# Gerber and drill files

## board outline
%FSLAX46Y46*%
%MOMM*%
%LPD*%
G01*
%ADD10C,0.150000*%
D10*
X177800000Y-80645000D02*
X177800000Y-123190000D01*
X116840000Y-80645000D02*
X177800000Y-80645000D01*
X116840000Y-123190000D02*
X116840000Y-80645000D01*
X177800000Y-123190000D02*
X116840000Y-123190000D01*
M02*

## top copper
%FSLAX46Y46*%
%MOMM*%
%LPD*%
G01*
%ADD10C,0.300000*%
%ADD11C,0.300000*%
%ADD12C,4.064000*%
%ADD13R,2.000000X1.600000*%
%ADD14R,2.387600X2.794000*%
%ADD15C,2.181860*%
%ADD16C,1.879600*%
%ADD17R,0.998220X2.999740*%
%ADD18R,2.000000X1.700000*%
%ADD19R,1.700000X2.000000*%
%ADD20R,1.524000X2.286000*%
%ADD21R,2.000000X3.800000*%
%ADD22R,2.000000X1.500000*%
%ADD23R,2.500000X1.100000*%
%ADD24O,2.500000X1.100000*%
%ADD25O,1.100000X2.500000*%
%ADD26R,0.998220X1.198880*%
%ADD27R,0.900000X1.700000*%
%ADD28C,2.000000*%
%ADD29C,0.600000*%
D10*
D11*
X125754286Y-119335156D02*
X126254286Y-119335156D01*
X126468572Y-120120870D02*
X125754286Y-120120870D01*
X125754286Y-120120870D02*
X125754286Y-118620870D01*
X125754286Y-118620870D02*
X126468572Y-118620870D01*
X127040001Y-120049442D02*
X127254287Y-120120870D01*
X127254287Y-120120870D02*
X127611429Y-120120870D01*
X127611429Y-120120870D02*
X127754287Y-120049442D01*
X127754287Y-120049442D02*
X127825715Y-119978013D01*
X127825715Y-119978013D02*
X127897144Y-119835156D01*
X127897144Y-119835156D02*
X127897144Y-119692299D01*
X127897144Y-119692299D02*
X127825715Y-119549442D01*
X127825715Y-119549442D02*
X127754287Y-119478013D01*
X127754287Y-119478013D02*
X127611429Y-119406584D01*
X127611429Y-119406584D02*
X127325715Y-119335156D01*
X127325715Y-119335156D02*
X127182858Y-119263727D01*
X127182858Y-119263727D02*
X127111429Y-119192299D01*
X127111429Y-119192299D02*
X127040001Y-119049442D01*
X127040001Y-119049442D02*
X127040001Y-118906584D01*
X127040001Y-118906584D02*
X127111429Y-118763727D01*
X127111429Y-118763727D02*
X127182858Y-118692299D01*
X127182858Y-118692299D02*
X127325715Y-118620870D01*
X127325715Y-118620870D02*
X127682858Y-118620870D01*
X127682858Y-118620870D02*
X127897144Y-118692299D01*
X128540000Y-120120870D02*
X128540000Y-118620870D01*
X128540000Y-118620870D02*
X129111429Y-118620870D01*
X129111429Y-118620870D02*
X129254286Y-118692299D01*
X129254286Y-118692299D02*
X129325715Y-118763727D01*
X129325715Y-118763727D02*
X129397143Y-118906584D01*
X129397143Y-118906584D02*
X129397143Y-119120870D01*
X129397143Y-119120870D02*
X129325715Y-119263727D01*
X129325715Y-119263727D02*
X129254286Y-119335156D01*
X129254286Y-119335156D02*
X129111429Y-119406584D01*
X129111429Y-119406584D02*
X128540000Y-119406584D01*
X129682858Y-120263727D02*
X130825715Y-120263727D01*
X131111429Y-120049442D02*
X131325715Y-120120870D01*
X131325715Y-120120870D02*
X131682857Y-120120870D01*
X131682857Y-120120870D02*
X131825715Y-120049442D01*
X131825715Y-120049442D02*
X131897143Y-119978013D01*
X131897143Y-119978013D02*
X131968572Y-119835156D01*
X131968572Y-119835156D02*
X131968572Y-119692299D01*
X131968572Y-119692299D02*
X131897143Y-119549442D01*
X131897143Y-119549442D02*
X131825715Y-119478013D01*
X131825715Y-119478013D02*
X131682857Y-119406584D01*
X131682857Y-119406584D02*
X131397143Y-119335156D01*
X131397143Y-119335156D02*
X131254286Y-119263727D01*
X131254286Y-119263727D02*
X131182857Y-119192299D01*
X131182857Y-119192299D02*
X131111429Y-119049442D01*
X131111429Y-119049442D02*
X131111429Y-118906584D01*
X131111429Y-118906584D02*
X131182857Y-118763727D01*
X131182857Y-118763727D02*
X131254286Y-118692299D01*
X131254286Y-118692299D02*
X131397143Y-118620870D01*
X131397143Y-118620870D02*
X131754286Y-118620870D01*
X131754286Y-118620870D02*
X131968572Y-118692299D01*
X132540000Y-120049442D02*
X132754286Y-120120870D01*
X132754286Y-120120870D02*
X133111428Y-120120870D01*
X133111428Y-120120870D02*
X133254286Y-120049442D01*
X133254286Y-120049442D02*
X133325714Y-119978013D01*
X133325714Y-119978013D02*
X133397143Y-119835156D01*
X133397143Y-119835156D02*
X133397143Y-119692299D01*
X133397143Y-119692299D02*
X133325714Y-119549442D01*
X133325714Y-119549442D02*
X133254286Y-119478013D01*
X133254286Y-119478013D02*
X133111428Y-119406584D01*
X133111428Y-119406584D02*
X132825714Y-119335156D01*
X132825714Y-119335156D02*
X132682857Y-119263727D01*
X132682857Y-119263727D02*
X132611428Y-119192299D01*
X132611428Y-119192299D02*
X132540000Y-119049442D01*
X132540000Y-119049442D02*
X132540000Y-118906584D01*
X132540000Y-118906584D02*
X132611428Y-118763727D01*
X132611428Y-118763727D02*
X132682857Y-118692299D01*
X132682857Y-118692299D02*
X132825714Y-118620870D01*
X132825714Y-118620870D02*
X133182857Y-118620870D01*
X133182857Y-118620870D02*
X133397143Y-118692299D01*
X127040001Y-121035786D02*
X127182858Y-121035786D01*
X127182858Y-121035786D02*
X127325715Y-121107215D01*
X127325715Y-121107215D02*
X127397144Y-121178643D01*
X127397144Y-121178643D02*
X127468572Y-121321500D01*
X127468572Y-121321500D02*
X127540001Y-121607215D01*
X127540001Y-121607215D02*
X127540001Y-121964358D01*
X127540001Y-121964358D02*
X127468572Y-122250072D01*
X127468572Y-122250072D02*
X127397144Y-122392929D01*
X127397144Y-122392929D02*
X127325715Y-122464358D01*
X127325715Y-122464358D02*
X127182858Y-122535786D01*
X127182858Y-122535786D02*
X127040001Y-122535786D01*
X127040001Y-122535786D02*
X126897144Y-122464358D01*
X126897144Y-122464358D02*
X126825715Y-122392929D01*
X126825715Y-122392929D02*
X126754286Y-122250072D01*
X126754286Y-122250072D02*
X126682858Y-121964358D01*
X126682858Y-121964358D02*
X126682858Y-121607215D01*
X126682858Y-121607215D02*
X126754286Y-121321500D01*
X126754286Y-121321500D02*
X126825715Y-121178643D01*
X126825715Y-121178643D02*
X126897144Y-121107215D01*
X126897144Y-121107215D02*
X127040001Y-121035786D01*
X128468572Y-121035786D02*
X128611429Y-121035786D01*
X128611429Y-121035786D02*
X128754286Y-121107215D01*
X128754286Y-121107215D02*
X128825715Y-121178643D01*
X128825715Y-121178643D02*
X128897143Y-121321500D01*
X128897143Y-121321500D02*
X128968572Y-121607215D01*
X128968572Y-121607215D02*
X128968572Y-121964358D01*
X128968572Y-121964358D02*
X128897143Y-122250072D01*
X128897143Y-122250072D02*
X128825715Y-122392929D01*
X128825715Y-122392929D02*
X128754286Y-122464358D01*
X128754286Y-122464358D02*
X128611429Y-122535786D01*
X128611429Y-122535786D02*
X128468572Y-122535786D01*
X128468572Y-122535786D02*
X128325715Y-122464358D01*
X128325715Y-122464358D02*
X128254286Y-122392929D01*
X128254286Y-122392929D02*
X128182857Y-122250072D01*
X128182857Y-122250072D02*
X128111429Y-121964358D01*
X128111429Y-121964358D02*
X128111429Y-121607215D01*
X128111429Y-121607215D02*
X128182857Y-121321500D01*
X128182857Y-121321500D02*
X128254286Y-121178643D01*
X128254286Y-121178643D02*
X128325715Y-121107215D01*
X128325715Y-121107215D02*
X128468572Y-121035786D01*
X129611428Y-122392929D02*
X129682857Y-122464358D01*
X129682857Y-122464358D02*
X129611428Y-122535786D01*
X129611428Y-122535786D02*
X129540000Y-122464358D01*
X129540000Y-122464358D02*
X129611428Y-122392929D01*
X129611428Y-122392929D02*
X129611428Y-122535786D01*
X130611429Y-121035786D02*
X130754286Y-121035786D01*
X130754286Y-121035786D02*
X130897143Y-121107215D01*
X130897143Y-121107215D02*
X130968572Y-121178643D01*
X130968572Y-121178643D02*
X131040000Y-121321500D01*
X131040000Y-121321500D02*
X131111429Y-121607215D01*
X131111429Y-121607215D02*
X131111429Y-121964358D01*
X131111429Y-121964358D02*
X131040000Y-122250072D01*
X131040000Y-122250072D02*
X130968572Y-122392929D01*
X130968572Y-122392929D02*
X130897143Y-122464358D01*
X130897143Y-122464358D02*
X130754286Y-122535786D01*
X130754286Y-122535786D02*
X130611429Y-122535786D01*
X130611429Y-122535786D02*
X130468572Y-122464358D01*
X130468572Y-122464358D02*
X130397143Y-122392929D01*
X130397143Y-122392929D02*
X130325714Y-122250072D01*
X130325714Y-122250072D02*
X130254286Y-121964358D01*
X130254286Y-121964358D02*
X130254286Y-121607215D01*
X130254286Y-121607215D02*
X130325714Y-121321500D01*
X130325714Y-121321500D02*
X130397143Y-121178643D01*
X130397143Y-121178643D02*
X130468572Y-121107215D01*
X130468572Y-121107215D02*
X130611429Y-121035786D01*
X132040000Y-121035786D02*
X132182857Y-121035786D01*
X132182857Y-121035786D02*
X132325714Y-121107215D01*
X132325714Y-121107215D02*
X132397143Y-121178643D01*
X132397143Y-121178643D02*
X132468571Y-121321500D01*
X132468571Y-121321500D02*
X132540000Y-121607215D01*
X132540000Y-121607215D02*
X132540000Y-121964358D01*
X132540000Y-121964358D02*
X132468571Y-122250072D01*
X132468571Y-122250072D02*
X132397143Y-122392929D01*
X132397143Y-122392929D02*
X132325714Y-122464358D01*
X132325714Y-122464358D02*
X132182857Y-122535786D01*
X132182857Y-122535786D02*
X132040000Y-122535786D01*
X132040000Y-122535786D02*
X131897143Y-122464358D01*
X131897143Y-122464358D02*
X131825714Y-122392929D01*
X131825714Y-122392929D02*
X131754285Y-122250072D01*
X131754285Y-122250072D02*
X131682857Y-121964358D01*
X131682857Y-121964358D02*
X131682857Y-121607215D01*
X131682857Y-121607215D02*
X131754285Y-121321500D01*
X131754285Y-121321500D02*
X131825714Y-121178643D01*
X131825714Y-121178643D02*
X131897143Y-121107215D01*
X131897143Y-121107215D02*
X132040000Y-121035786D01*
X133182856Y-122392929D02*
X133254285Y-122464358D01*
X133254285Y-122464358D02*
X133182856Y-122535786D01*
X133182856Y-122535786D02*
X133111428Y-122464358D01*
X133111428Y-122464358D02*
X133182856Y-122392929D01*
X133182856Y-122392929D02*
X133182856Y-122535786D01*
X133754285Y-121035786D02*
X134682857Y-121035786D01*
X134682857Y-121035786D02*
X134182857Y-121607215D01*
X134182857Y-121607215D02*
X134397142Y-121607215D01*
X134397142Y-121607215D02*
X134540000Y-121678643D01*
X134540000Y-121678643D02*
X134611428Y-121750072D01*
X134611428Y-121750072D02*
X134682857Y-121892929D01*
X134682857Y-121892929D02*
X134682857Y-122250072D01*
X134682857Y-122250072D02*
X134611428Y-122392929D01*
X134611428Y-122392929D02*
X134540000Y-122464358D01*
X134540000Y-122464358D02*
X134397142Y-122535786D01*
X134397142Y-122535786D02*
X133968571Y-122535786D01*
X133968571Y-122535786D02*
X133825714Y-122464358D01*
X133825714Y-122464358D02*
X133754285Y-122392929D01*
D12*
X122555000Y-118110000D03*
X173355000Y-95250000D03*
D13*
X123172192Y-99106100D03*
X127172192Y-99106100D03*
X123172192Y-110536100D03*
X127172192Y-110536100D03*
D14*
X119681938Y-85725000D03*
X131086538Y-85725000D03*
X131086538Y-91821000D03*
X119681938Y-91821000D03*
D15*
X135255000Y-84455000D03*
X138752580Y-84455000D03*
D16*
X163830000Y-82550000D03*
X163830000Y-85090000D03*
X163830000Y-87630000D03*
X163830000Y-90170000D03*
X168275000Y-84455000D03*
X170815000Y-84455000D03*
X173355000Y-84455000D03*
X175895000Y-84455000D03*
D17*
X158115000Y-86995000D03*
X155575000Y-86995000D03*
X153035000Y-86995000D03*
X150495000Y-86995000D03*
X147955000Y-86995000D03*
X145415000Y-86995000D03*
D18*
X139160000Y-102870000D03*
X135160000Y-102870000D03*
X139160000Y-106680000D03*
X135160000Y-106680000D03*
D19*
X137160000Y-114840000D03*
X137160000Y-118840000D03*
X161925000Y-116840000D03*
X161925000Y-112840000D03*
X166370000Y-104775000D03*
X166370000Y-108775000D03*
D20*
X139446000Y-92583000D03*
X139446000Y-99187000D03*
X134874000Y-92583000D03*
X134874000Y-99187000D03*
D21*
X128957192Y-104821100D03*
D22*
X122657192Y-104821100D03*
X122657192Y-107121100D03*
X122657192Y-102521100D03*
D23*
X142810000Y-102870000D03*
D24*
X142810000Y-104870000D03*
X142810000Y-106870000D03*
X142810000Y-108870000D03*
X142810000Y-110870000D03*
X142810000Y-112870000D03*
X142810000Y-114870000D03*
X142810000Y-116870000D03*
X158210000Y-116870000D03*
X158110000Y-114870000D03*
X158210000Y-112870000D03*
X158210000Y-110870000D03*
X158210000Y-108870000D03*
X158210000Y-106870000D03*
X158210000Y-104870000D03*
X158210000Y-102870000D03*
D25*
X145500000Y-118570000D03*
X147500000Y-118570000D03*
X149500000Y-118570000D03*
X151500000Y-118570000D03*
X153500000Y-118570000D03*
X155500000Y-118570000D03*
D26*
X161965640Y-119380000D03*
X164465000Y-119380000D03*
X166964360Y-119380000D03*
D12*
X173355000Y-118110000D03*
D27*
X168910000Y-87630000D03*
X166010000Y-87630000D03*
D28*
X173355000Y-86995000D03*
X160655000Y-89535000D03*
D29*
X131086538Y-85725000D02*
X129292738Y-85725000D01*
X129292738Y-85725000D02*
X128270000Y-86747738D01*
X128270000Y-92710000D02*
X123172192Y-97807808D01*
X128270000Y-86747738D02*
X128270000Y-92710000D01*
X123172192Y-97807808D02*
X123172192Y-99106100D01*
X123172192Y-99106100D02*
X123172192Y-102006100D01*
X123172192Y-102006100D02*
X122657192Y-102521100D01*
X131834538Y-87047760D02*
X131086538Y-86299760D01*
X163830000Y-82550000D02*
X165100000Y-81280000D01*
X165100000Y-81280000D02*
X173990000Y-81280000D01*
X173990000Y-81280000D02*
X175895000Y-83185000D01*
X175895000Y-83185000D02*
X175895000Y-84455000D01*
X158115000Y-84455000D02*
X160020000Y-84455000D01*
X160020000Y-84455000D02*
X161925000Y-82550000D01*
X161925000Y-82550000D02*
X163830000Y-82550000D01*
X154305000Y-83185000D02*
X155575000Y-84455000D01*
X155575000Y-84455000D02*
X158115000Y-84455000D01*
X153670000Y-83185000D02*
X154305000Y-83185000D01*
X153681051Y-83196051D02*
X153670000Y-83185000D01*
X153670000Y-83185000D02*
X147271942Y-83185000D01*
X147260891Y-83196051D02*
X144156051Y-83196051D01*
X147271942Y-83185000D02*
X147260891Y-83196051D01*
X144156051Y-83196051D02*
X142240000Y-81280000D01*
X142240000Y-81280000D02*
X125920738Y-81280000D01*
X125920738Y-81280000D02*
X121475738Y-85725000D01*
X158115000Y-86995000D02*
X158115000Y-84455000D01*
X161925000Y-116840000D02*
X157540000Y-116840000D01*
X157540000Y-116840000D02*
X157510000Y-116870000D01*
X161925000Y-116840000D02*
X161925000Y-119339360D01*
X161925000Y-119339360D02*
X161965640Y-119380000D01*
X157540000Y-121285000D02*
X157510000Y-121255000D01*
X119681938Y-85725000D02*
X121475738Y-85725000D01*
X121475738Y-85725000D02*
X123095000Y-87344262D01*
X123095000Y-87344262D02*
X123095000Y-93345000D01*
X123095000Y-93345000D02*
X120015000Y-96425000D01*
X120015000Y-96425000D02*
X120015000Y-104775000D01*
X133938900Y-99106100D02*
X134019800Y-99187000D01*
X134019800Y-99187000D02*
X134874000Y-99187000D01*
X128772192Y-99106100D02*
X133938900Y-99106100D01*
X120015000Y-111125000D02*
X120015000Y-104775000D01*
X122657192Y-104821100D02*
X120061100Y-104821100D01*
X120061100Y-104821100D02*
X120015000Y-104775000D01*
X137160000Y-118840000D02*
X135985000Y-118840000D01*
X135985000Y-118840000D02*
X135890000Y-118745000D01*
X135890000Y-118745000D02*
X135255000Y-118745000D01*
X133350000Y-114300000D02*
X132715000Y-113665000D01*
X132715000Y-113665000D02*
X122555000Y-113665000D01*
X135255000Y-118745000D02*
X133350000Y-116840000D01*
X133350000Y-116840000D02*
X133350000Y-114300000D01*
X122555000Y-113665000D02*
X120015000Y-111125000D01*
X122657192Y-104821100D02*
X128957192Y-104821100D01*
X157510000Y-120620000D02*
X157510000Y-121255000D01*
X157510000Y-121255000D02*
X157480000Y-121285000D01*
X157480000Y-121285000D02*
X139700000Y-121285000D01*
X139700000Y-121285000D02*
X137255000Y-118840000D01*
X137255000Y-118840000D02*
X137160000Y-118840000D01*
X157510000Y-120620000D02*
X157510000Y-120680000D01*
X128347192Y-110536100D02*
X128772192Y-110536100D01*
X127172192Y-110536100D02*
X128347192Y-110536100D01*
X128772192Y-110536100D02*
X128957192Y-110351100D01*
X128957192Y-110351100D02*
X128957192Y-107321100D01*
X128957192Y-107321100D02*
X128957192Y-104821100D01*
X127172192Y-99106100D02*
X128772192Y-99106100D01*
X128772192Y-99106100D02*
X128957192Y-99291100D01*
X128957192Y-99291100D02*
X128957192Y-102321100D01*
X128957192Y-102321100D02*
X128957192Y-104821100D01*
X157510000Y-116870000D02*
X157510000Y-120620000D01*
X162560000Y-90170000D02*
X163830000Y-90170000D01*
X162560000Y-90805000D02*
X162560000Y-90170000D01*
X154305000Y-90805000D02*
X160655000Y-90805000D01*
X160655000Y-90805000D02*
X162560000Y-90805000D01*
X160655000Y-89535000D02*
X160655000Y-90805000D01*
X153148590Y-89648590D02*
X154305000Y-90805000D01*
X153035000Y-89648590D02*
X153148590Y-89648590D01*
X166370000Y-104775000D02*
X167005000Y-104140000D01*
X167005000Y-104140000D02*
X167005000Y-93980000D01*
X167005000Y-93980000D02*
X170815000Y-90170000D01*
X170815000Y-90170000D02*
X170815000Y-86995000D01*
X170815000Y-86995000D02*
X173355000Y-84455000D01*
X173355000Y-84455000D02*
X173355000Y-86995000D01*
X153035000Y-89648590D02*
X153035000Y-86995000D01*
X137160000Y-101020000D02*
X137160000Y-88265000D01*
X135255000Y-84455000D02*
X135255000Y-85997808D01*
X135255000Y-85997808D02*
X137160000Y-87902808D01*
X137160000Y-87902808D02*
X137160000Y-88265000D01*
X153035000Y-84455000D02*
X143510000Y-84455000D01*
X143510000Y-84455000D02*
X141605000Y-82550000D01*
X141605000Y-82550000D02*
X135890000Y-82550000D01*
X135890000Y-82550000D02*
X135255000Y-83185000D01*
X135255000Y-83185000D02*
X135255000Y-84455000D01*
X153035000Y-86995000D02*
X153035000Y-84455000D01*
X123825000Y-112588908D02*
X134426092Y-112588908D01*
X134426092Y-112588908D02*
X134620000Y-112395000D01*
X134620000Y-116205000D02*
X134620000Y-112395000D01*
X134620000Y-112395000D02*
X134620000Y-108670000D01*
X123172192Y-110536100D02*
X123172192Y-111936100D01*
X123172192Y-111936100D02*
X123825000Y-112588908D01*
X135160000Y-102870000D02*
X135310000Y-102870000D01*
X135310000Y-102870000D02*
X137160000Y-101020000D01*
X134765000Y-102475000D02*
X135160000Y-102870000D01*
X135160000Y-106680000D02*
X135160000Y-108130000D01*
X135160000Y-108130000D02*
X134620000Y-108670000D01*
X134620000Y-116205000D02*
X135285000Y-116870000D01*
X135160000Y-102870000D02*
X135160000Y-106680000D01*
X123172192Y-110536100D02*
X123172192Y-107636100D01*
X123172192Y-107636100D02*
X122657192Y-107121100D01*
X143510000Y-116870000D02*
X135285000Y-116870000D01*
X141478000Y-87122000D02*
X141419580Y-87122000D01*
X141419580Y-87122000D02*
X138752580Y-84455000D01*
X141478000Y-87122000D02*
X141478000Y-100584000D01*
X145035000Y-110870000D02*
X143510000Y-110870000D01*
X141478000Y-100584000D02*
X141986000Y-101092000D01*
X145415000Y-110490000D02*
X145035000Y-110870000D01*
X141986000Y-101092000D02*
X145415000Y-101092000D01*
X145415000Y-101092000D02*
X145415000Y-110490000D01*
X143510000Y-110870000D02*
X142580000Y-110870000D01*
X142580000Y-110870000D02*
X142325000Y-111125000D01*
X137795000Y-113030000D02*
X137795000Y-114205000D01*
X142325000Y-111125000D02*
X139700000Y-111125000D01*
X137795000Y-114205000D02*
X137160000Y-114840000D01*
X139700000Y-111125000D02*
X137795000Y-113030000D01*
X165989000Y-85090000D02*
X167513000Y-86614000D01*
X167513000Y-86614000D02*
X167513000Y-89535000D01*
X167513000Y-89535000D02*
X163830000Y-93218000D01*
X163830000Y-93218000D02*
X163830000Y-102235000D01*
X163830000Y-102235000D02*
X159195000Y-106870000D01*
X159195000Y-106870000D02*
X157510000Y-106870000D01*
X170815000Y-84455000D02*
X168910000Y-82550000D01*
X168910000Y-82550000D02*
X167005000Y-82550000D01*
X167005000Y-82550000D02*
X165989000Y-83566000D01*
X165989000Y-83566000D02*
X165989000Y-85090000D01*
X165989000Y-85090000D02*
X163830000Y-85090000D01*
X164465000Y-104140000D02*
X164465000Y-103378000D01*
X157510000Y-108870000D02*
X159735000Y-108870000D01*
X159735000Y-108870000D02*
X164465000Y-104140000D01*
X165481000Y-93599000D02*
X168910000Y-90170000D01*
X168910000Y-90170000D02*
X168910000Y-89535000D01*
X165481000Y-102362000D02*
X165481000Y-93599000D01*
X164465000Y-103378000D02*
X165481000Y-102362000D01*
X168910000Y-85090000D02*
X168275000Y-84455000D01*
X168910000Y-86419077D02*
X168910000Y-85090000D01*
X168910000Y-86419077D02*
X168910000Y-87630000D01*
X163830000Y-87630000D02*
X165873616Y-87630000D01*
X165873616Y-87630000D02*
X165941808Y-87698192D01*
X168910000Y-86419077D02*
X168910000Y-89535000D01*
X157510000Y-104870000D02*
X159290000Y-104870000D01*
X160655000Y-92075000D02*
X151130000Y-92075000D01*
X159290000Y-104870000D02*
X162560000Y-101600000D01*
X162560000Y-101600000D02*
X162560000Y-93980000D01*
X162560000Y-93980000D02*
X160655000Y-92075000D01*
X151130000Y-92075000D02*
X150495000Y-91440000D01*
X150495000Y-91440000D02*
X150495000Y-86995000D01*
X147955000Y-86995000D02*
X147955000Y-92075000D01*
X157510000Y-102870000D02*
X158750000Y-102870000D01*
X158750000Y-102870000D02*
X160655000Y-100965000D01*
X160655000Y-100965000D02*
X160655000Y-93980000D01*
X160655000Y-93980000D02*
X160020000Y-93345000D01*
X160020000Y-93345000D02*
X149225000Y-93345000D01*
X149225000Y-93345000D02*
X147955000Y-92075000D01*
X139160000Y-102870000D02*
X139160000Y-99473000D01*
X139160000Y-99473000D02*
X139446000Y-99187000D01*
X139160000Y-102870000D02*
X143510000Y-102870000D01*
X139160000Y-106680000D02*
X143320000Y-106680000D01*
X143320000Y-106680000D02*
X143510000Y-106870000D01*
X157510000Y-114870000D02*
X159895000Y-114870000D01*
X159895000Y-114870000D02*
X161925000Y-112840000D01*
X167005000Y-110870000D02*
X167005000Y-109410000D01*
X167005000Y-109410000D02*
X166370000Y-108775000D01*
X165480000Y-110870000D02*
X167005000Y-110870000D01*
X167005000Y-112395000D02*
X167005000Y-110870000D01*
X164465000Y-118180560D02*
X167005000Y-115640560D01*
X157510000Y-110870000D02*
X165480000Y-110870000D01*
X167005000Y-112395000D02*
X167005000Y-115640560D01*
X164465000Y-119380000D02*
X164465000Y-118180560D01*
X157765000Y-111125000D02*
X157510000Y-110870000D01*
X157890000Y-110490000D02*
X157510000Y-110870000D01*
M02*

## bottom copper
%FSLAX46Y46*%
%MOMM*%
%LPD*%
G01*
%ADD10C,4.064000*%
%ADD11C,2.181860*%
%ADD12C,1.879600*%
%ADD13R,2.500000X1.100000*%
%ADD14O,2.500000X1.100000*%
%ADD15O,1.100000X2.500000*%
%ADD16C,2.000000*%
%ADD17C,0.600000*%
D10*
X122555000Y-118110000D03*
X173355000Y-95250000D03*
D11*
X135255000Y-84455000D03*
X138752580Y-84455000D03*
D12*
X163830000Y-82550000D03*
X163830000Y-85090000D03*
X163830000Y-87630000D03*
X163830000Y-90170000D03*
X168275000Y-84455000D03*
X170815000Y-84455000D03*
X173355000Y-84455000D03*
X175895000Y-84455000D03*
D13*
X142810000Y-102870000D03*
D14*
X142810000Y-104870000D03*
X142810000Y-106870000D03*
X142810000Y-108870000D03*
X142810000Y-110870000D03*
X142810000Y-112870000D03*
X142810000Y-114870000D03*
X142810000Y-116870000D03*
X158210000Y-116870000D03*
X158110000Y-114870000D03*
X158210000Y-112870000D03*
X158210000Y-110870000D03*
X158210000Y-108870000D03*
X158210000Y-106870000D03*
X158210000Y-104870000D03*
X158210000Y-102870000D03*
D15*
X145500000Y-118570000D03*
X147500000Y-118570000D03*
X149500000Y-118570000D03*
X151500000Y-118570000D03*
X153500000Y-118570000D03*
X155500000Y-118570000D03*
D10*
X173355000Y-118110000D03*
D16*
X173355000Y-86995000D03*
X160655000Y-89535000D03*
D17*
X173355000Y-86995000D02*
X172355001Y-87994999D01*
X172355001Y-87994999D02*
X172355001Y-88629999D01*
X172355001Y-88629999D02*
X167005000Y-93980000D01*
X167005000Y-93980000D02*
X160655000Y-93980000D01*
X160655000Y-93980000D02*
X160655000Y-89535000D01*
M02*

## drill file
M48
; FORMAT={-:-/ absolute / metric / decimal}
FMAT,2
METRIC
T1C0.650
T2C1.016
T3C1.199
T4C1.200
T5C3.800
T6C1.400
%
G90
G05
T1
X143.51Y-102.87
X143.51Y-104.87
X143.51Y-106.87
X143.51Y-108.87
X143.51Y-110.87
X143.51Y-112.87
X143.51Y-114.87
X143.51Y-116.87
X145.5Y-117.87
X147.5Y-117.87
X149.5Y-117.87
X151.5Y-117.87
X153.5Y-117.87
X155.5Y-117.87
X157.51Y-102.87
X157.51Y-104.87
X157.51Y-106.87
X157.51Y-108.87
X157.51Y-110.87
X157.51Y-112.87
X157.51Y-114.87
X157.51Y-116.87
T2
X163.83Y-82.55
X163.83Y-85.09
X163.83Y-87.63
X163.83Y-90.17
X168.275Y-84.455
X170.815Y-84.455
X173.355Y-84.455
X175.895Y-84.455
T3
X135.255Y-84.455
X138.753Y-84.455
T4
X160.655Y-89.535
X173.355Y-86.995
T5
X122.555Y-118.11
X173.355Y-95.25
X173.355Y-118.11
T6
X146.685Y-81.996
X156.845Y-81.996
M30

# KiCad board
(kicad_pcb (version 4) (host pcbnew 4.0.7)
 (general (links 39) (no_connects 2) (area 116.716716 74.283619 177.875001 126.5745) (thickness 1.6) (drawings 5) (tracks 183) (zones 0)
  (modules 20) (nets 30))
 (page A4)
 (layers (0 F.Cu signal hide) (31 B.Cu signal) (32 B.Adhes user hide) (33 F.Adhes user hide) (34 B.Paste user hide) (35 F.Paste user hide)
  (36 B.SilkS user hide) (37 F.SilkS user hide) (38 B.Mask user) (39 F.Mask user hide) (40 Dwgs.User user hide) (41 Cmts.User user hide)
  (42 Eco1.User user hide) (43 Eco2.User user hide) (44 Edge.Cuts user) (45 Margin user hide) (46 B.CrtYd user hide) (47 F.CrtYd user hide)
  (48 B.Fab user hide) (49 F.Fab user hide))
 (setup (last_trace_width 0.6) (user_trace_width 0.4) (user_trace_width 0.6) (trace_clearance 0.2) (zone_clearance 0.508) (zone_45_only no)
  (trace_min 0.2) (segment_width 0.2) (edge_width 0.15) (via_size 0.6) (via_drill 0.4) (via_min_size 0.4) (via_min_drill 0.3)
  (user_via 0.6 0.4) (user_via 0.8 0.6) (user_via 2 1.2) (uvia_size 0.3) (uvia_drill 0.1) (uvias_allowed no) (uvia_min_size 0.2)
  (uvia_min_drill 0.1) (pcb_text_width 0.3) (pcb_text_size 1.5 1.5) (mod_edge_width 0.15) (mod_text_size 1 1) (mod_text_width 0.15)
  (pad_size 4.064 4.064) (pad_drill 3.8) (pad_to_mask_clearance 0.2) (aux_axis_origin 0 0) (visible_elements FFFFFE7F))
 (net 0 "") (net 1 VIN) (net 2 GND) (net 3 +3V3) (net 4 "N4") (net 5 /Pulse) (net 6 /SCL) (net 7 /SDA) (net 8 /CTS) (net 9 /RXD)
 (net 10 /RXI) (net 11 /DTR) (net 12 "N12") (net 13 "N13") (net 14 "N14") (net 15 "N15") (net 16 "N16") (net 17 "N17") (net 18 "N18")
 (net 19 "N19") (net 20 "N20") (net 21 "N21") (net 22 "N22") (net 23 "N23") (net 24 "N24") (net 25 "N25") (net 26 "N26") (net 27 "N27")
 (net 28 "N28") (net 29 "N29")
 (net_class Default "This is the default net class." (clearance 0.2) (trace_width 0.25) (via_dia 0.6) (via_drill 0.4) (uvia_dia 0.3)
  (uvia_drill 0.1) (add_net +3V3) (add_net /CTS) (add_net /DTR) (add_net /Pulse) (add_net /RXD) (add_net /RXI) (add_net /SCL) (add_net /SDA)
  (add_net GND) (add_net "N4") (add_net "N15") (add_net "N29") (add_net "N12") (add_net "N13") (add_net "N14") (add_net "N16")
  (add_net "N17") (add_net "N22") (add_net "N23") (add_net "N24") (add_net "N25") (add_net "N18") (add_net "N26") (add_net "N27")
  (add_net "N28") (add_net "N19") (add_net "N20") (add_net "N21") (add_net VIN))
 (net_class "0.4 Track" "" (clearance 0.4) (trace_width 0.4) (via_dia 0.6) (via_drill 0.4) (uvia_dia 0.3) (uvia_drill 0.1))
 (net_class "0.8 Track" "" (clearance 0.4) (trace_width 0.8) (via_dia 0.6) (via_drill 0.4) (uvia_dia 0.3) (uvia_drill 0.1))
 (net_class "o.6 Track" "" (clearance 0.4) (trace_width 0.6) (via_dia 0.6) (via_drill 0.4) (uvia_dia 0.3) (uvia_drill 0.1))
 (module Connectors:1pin (layer F.Cu) (at 122.555 118.11)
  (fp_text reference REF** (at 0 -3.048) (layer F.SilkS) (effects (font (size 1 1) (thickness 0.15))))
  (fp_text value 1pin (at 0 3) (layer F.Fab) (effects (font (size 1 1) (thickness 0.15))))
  (pad 1 thru_hole circle (at 0 0) (size 4.064 4.064) (drill 3.8) (layers *.Cu *.Mask)))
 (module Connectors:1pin (layer F.Cu) (at 173.355 95.25)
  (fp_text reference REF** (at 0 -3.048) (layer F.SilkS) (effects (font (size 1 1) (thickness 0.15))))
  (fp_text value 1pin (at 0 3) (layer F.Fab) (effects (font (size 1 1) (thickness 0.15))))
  (pad 1 thru_hole circle (at 0 0) (size 4.064 4.064) (drill 3.8) (layers *.Cu *.Mask)))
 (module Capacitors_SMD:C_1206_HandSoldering (layer F.Cu) (at 125.172192 99.1061)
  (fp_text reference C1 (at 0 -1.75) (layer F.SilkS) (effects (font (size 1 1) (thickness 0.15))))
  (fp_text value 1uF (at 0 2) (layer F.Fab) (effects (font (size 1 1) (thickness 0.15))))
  (pad 1 smd rect (at -2 0) (size 2 1.6) (layers F.Cu F.Paste F.Mask) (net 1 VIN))
  (pad 2 smd rect (at 2 0) (size 2 1.6) (layers F.Cu F.Paste F.Mask) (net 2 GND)))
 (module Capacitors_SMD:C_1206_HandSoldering (layer F.Cu) (at 125.172192 110.5361)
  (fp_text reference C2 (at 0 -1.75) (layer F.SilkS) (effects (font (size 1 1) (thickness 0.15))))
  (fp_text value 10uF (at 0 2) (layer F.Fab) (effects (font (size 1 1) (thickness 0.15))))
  (pad 1 smd rect (at -2 0) (size 2 1.6) (layers F.Cu F.Paste F.Mask) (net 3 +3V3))
  (pad 2 smd rect (at 2 0) (size 2 1.6) (layers F.Cu F.Paste F.Mask) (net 2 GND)))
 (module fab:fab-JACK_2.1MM (layer F.Cu) (at 125.447738 88.138 180)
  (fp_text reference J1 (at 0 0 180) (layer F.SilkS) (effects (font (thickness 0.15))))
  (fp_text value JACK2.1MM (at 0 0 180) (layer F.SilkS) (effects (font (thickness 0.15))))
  (pad CONT smd rect (at 5.7658 2.413 180) (size 2.3876 2.794) (layers F.Cu F.Paste F.Mask) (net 2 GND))
  (pad PIN smd rect (at -5.6388 2.413 180) (size 2.3876 2.794) (layers F.Cu F.Paste F.Mask) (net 1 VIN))
  (pad PIN1 smd rect (at -5.6388 -3.683 180) (size 2.3876 2.794) (layers F.Cu F.Paste F.Mask))
  (pad SHUN smd rect (at 5.7658 -3.683 180) (size 2.3876 2.794) (layers F.Cu F.Paste F.Mask) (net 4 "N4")))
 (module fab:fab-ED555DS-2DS (layer F.Cu) (at 137.05332 84.455 180)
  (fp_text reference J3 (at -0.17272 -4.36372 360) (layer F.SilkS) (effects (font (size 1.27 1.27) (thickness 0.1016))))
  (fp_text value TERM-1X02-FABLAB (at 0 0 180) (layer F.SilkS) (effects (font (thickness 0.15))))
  (pad 1 thru_hole circle (at 1.79832 0 180) (size 2.18186 2.18186) (drill 1.19888) (layers *.Cu F.Paste F.SilkS F.Mask) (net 3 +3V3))
  (pad 2 thru_hole circle (at -1.69926 0 180) (size 2.18186 2.18186) (drill 1.19888) (layers *.Cu F.Paste F.SilkS F.Mask) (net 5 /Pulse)))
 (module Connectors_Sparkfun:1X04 (layer F.Cu) (at 163.83 82.55 270)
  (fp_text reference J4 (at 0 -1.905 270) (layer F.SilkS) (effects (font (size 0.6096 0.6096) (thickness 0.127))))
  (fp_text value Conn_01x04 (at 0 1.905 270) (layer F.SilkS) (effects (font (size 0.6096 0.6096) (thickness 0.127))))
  (pad 1 thru_hole circle (at 0 0 270) (size 1.8796 1.8796) (drill 1.016) (layers *.Cu *.Mask) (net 2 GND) (solder_mask_margin 0.1016))
  (pad 2 thru_hole circle (at 2.54 0 270) (size 1.8796 1.8796) (drill 1.016) (layers *.Cu *.Mask) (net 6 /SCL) (solder_mask_margin 0.1016))
  (pad 3 thru_hole circle (at 5.08 0 270) (size 1.8796 1.8796) (drill 1.016) (layers *.Cu *.Mask) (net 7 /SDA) (solder_mask_margin 0.1016))
  (pad 4 thru_hole circle (at 7.62 0 270) (size 1.8796 1.8796) (drill 1.016) (layers *.Cu *.Mask) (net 3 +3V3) (solder_mask_margin 0.1016)))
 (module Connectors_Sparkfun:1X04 (layer F.Cu) (at 168.275 84.455)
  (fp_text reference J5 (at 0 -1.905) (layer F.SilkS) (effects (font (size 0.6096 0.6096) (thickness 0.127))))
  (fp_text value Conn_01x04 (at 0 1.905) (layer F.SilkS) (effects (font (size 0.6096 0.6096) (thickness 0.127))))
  (pad 1 thru_hole circle (at 0 0) (size 1.8796 1.8796) (drill 1.016) (layers *.Cu *.Mask) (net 7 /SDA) (solder_mask_margin 0.1016))
  (pad 2 thru_hole circle (at 2.54 0) (size 1.8796 1.8796) (drill 1.016) (layers *.Cu *.Mask) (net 6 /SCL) (solder_mask_margin 0.1016))
  (pad 3 thru_hole circle (at 5.08 0) (size 1.8796 1.8796) (drill 1.016) (layers *.Cu *.Mask) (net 3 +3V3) (solder_mask_margin 0.1016))
  (pad 4 thru_hole circle (at 7.62 0) (size 1.8796 1.8796) (drill 1.016) (layers *.Cu *.Mask) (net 2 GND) (solder_mask_margin 0.1016)))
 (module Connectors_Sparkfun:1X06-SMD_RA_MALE (layer F.Cu) (at 151.765 81.99628 180)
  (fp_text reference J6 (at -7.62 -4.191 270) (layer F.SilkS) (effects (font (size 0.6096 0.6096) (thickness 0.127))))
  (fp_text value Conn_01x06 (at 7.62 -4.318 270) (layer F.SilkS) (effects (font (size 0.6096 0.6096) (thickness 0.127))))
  (pad 1 smd rect (at -6.35 -4.99872 270) (size 2.99974 0.99822) (layers F.Cu F.Paste F.Mask) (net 2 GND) (solder_mask_margin 0.1016))
  (pad 2 smd rect (at -3.81 -4.99872 270) (size 2.99974 0.99822) (layers F.Cu F.Paste F.Mask) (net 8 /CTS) (solder_mask_margin 0.1016))
  (pad 3 smd rect (at -1.27 -4.99872 270) (size 2.99974 0.99822) (layers F.Cu F.Paste F.Mask) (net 3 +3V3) (solder_mask_margin 0.1016))
  (pad 4 smd rect (at 1.27 -4.99872 270) (size 2.99974 0.99822) (layers F.Cu F.Paste F.Mask) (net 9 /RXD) (solder_mask_margin 0.1016))
  (pad 5 smd rect (at 3.81 -4.99872 270) (size 2.99974 0.99822) (layers F.Cu F.Paste F.Mask) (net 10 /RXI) (solder_mask_margin 0.1016))
  (pad 6 smd rect (at 6.35 -4.99872 270) (size 2.99974 0.99822) (layers F.Cu F.Paste F.Mask) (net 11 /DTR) (solder_mask_margin 0.1016))
  (pad "" np_thru_hole circle (at -5.08 0 180) (size 1.39954 1.39954) (drill 1.39954) (layers *.Cu *.Mask) (solder_mask_margin 0.1016))
  (pad "" np_thru_hole circle (at 5.08 0 180) (size 1.39954 1.39954) (drill 1.39954) (layers *.Cu *.Mask) (solder_mask_margin 0.1016)))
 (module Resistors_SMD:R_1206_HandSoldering (layer F.Cu) (at 137.16 102.87 180)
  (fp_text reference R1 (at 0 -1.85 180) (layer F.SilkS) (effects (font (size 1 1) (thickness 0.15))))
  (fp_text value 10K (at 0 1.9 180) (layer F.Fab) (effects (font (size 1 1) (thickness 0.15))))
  (pad 1 smd rect (at -2 0 180) (size 2 1.7) (layers F.Cu F.Paste F.Mask) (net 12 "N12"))
  (pad 2 smd rect (at 2 0 180) (size 2 1.7) (layers F.Cu F.Paste F.Mask) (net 3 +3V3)))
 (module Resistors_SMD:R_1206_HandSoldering (layer F.Cu) (at 137.16 106.68 180)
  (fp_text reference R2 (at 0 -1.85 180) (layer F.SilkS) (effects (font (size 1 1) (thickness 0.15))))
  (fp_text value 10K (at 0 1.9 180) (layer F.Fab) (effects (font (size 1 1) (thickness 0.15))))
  (pad 1 smd rect (at -2 0 180) (size 2 1.7) (layers F.Cu F.Paste F.Mask) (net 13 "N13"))
  (pad 2 smd rect (at 2 0 180) (size 2 1.7) (layers F.Cu F.Paste F.Mask) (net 3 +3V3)))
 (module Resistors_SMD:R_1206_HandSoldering (layer F.Cu) (at 137.16 116.84 270)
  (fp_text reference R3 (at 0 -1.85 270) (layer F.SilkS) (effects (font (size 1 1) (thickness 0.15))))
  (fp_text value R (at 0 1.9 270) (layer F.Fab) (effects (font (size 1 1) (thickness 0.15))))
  (pad 1 smd rect (at -2 0 270) (size 2 1.7) (layers F.Cu F.Paste F.Mask) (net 5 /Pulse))
  (pad 2 smd rect (at 2 0 270) (size 2 1.7) (layers F.Cu F.Paste F.Mask) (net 2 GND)))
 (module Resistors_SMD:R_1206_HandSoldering (layer F.Cu) (at 161.925 114.84 90)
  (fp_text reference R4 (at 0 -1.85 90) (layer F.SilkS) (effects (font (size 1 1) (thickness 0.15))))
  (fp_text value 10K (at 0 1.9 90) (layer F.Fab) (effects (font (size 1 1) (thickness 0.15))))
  (pad 1 smd rect (at -2 0 90) (size 2 1.7) (layers F.Cu F.Paste F.Mask) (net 2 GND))
  (pad 2 smd rect (at 2 0 90) (size 2 1.7) (layers F.Cu F.Paste F.Mask) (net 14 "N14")))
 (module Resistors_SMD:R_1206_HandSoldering (layer F.Cu) (at 166.37 106.775 270)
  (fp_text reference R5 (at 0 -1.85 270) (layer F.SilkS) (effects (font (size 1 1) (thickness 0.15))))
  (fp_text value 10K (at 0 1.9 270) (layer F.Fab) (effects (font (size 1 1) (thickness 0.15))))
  (pad 1 smd rect (at -2 0 270) (size 2 1.7) (layers F.Cu F.Paste F.Mask) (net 3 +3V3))
  (pad 2 smd rect (at 2 0 270) (size 2 1.7) (layers F.Cu F.Paste F.Mask) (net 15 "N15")))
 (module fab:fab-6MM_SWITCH (layer F.Cu) (at 137.16 95.885 270)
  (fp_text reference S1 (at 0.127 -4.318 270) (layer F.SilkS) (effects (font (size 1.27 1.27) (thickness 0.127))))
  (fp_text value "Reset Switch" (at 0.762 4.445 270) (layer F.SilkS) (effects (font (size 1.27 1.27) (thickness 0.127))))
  (pad 1 smd rect (at -3.302 -2.286 270) (size 2.286 1.524) (layers F.Cu F.Paste F.Mask) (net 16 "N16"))
  (pad 2 smd rect (at 3.302 -2.286 270) (size 2.286 1.524) (layers F.Cu F.Paste F.Mask) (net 12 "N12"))
  (pad 3 smd rect (at -3.302 2.286 270) (size 2.286 1.524) (layers F.Cu F.Paste F.Mask) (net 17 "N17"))
  (pad 4 smd rect (at 3.302 2.286 270) (size 2.286 1.524) (layers F.Cu F.Paste F.Mask) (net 2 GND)))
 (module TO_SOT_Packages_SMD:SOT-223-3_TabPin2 (layer F.Cu) (at 125.807192 104.8211)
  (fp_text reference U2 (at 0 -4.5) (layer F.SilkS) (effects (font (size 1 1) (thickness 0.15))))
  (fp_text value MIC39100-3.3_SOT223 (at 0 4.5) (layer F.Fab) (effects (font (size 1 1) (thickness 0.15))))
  (pad 2 smd rect (at 3.15 0) (size 2 3.8) (layers F.Cu F.Paste F.Mask) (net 2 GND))
  (pad 2 smd rect (at -3.15 0) (size 2 1.5) (layers F.Cu F.Paste F.Mask) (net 2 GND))
  (pad 3 smd rect (at -3.15 2.3) (size 2 1.5) (layers F.Cu F.Paste F.Mask) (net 3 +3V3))
  (pad 1 smd rect (at -3.15 -2.3) (size 2 1.5) (layers F.Cu F.Paste F.Mask) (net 1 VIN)))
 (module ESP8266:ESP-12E (layer F.Cu) (at 143.51 102.87)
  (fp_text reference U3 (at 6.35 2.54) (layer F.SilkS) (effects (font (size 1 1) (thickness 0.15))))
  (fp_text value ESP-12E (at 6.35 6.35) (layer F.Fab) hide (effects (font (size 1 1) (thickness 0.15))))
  (pad 1 thru_hole rect (at 0 0) (size 2.5 1.1) (drill 0.65 (offset -0.7 0)) (layers *.Cu *.Mask F.SilkS) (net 12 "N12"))
  (pad 2 thru_hole oval (at 0 2) (size 2.5 1.1) (drill 0.65 (offset -0.7 0)) (layers *.Cu *.Mask F.SilkS) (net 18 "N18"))
  (pad 3 thru_hole oval (at 0 4) (size 2.5 1.1) (drill 0.65 (offset -0.7 0)) (layers *.Cu *.Mask F.SilkS) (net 13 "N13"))
  (pad 4 thru_hole oval (at 0 6) (size 2.5 1.1) (drill 0.65 (offset -0.7 0)) (layers *.Cu *.Mask F.SilkS) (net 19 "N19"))
  (pad 5 thru_hole oval (at 0 8) (size 2.5 1.1) (drill 0.65 (offset -0.7 0)) (layers *.Cu *.Mask F.SilkS) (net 5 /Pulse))
  (pad 6 thru_hole oval (at 0 10) (size 2.5 1.1) (drill 0.65 (offset -0.7 0)) (layers *.Cu *.Mask F.SilkS) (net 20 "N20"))
  (pad 7 thru_hole oval (at 0 12) (size 2.5 1.1) (drill 0.65 (offset -0.7 0)) (layers *.Cu *.Mask F.SilkS) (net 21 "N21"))
  (pad 8 thru_hole oval (at 0 14) (size 2.5 1.1) (drill 0.65 (offset -0.7 0)) (layers *.Cu *.Mask F.SilkS) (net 3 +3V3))
  (pad 9 thru_hole oval (at 14 14) (size 2.5 1.1) (drill 0.65 (offset 0.7 0)) (layers *.Cu *.Mask F.SilkS) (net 2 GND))
  (pad 10 thru_hole oval (at 14 12) (size 2.5 1.1) (drill 0.65 (offset 0.6 0)) (layers *.Cu *.Mask F.SilkS) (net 14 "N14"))
  (pad 11 thru_hole oval (at 14 10) (size 2.5 1.1) (drill 0.65 (offset 0.7 0)) (layers *.Cu *.Mask F.SilkS) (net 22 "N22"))
  (pad 12 thru_hole oval (at 14 8) (size 2.5 1.1) (drill 0.65 (offset 0.7 0)) (layers *.Cu *.Mask F.SilkS) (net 15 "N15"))
  (pad 13 thru_hole oval (at 14 6) (size 2.5 1.1) (drill 0.65 (offset 0.7 0)) (layers *.Cu *.Mask F.SilkS) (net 7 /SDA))
  (pad 14 thru_hole oval (at 14 4) (size 2.5 1.1) (drill 0.65 (offset 0.7 0)) (layers *.Cu *.Mask F.SilkS) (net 6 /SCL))
  (pad 15 thru_hole oval (at 14 2) (size 2.5 1.1) (drill 0.65 (offset 0.7 0)) (layers *.Cu *.Mask F.SilkS) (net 9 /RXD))
  (pad 16 thru_hole oval (at 14 0) (size 2.5 1.1) (drill 0.65 (offset 0.7 0)) (layers *.Cu *.Mask F.SilkS) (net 10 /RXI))
  (pad 17 thru_hole oval (at 1.99 15 90) (size 2.5 1.1) (drill 0.65 (offset -0.7 0)) (layers *.Cu *.Mask F.SilkS) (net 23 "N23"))
  (pad 18 thru_hole oval (at 3.99 15 90) (size 2.5 1.1) (drill 0.65 (offset -0.7 0)) (layers *.Cu *.Mask F.SilkS) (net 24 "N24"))
  (pad 19 thru_hole oval (at 5.99 15 90) (size 2.5 1.1) (drill 0.65 (offset -0.7 0)) (layers *.Cu *.Mask F.SilkS) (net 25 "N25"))
  (pad 20 thru_hole oval (at 7.99 15 90) (size 2.5 1.1) (drill 0.65 (offset -0.7 0)) (layers *.Cu *.Mask F.SilkS) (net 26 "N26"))
  (pad 21 thru_hole oval (at 9.99 15 90) (size 2.5 1.1) (drill 0.65 (offset -0.7 0)) (layers *.Cu *.Mask F.SilkS) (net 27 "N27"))
  (pad 22 thru_hole oval (at 11.99 15 90) (size 2.5 1.1) (drill 0.65 (offset -0.7 0)) (layers *.Cu *.Mask F.SilkS) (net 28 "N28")))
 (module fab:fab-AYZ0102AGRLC (layer F.Cu) (at 164.465 121.6787 180)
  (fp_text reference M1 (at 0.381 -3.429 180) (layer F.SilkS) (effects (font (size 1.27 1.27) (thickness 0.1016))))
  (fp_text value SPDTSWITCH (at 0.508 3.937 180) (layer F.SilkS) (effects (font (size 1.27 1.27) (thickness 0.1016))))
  (pad 1 smd rect (at 2.49936 2.2987 180) (size 0.99822 1.19888) (layers F.Cu F.Paste F.Mask) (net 2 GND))
  (pad 2 smd rect (at 0 2.2987 180) (size 0.99822 1.19888) (layers F.Cu F.Paste F.Mask) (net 15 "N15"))
  (pad 3 smd rect (at -2.49936 2.2987 180) (size 0.99822 1.19888) (layers F.Cu F.Paste F.Mask) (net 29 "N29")))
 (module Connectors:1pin (layer F.Cu) (at 173.355 118.11)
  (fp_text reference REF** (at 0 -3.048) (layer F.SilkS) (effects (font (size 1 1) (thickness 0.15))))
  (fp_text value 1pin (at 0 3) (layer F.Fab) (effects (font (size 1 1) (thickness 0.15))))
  (pad 1 thru_hole circle (at 0 0) (size 4.064 4.064) (drill 3.8) (layers *.Cu *.Mask)))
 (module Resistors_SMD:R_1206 (layer F.Cu) (at 167.46 87.63 180)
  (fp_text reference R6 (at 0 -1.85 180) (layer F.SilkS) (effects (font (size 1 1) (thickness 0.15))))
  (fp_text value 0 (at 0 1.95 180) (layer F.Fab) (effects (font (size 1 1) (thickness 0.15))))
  (pad 1 smd rect (at -1.45 0 180) (size 0.9 1.7) (layers F.Cu F.Paste F.Mask) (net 7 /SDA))
  (pad 2 smd rect (at 1.45 0 180) (size 0.9 1.7) (layers F.Cu F.Paste F.Mask) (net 7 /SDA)))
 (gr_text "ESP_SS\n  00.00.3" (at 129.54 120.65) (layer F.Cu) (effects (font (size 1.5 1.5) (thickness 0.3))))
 (gr_line (start 177.8 80.645) (end 177.8 123.19) (layer Edge.Cuts) (width 0.15))
 (gr_line (start 116.84 80.645) (end 177.8 80.645) (layer Edge.Cuts) (width 0.15))
 (gr_line (start 116.84 123.19) (end 116.84 80.645) (layer Edge.Cuts) (width 0.15))
 (gr_line (start 177.8 123.19) (end 116.84 123.19) (layer Edge.Cuts) (width 0.15))
 (segment (start 131.086538 85.725) (end 129.292738 85.725) (width 0.6) (layer F.Cu) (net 1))
 (segment (start 129.292738 85.725) (end 128.27 86.747738) (width 0.6) (layer F.Cu) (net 1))
 (segment (start 128.27 92.71) (end 123.172192 97.807808) (width 0.6) (layer F.Cu) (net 1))
 (segment (start 128.27 86.747738) (end 128.27 92.71) (width 0.6) (layer F.Cu) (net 1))
 (segment (start 123.172192 97.807808) (end 123.172192 99.1061) (width 0.6) (layer F.Cu) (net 1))
 (segment (start 123.172192 99.1061) (end 123.172192 102.0061) (width 0.6) (layer F.Cu) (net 1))
 (segment (start 123.172192 102.0061) (end 122.657192 102.5211) (width 0.6) (layer F.Cu) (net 1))
 (segment (start 131.834538 87.04776) (end 131.086538 86.29976) (width 0.6) (layer F.Cu) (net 1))
 (segment (start 163.83 82.55) (end 165.1 81.28) (width 0.6) (layer F.Cu) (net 2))
 (segment (start 165.1 81.28) (end 173.99 81.28) (width 0.6) (layer F.Cu) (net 2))
 (segment (start 173.99 81.28) (end 175.895 83.185) (width 0.6) (layer F.Cu) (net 2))
 (segment (start 175.895 83.185) (end 175.895 84.455) (width 0.6) (layer F.Cu) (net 2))
 (segment (start 158.115 84.455) (end 160.02 84.455) (width 0.6) (layer F.Cu) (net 2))
 (segment (start 160.02 84.455) (end 161.925 82.55) (width 0.6) (layer F.Cu) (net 2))
 (segment (start 161.925 82.55) (end 163.83 82.55) (width 0.6) (layer F.Cu) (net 2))
 (segment (start 154.305 83.185) (end 155.575 84.455) (width 0.6) (layer F.Cu) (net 2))
 (segment (start 155.575 84.455) (end 158.115 84.455) (width 0.6) (layer F.Cu) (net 2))
 (segment (start 153.67 83.185) (end 154.305 83.185) (width 0.6) (layer F.Cu) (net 2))
 (segment (start 153.681051 83.196051) (end 153.67 83.185) (width 0.6) (layer F.Cu) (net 2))
 (segment (start 153.67 83.185) (end 147.271942 83.185) (width 0.6) (layer F.Cu) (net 2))
 (segment (start 147.260891 83.196051) (end 144.156051 83.196051) (width 0.6) (layer F.Cu) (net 2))
 (segment (start 147.271942 83.185) (end 147.260891 83.196051) (width 0.6) (layer F.Cu) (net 2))
 (segment (start 144.156051 83.196051) (end 142.24 81.28) (width 0.6) (layer F.Cu) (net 2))
 (segment (start 142.24 81.28) (end 125.920738 81.28) (width 0.6) (layer F.Cu) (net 2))
 (segment (start 125.920738 81.28) (end 121.475738 85.725) (width 0.6) (layer F.Cu) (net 2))
 (segment (start 158.115 86.995) (end 158.115 84.455) (width 0.6) (layer F.Cu) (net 2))
 (segment (start 161.925 116.84) (end 157.54 116.84) (width 0.6) (layer F.Cu) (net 2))
 (segment (start 157.54 116.84) (end 157.51 116.87) (width 0.6) (layer F.Cu) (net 2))
 (segment (start 161.925 116.84) (end 161.925 119.33936) (width 0.6) (layer F.Cu) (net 2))
 (segment (start 161.925 119.33936) (end 161.96564 119.38) (width 0.6) (layer F.Cu) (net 2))
 (segment (start 157.54 121.285) (end 157.51 121.255) (width 0.6) (layer F.Cu) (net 2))
 (segment (start 119.681938 85.725) (end 121.475738 85.725) (width 0.6) (layer F.Cu) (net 2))
 (segment (start 121.475738 85.725) (end 123.095 87.344262) (width 0.6) (layer F.Cu) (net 2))
 (segment (start 123.095 87.344262) (end 123.095 93.345) (width 0.6) (layer F.Cu) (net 2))
 (segment (start 123.095 93.345) (end 120.015 96.425) (width 0.6) (layer F.Cu) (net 2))
 (segment (start 120.015 96.425) (end 120.015 104.775) (width 0.6) (layer F.Cu) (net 2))
 (segment (start 133.9389 99.1061) (end 134.0198 99.187) (width 0.6) (layer F.Cu) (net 2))
 (segment (start 134.0198 99.187) (end 134.874 99.187) (width 0.6) (layer F.Cu) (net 2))
 (segment (start 128.772192 99.1061) (end 133.9389 99.1061) (width 0.6) (layer F.Cu) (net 2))
 (segment (start 120.015 111.125) (end 120.015 104.775) (width 0.6) (layer F.Cu) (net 2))
 (segment (start 122.657192 104.8211) (end 120.0611 104.8211) (width 0.6) (layer F.Cu) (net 2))
 (segment (start 120.0611 104.8211) (end 120.015 104.775) (width 0.6) (layer F.Cu) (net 2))
 (segment (start 137.16 118.84) (end 135.985 118.84) (width 0.6) (layer F.Cu) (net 2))
 (segment (start 135.985 118.84) (end 135.89 118.745) (width 0.6) (layer F.Cu) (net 2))
 (segment (start 135.89 118.745) (end 135.255 118.745) (width 0.6) (layer F.Cu) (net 2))
 (segment (start 133.35 114.3) (end 132.715 113.665) (width 0.6) (layer F.Cu) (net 2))
 (segment (start 132.715 113.665) (end 122.555 113.665) (width 0.6) (layer F.Cu) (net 2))
 (segment (start 135.255 118.745) (end 133.35 116.84) (width 0.6) (layer F.Cu) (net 2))
 (segment (start 133.35 116.84) (end 133.35 114.3) (width 0.6) (layer F.Cu) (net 2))
 (segment (start 122.555 113.665) (end 120.015 111.125) (width 0.6) (layer F.Cu) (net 2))
 (segment (start 122.657192 104.8211) (end 128.957192 104.8211) (width 0.6) (layer F.Cu) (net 2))
 (segment (start 157.51 120.62) (end 157.51 121.255) (width 0.6) (layer F.Cu) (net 2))
 (segment (start 157.51 121.255) (end 157.48 121.285) (width 0.6) (layer F.Cu) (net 2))
 (segment (start 157.48 121.285) (end 139.7 121.285) (width 0.6) (layer F.Cu) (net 2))
 (segment (start 139.7 121.285) (end 137.255 118.84) (width 0.6) (layer F.Cu) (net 2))
 (segment (start 137.255 118.84) (end 137.16 118.84) (width 0.6) (layer F.Cu) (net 2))
 (segment (start 157.51 120.62) (end 157.51 120.68) (width 0.6) (layer F.Cu) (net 2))
 (segment (start 128.347192 110.5361) (end 128.772192 110.5361) (width 0.6) (layer F.Cu) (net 2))
 (segment (start 127.172192 110.5361) (end 128.347192 110.5361) (width 0.6) (layer F.Cu) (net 2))
 (segment (start 128.772192 110.5361) (end 128.957192 110.3511) (width 0.6) (layer F.Cu) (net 2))
 (segment (start 128.957192 110.3511) (end 128.957192 107.3211) (width 0.6) (layer F.Cu) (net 2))
 (segment (start 128.957192 107.3211) (end 128.957192 104.8211) (width 0.6) (layer F.Cu) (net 2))
 (segment (start 127.172192 99.1061) (end 128.772192 99.1061) (width 0.6) (layer F.Cu) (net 2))
 (segment (start 128.772192 99.1061) (end 128.957192 99.2911) (width 0.6) (layer F.Cu) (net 2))
 (segment (start 128.957192 99.2911) (end 128.957192 102.3211) (width 0.6) (layer F.Cu) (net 2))
 (segment (start 128.957192 102.3211) (end 128.957192 104.8211) (width 0.6) (layer F.Cu) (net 2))
 (segment (start 157.51 116.87) (end 157.51 120.62) (width 0.6) (layer F.Cu) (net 2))
 (segment (start 162.56 90.17) (end 163.83 90.17) (width 0.6) (layer F.Cu) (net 3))
 (segment (start 162.56 90.805) (end 162.56 90.17) (width 0.6) (layer F.Cu) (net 3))
 (segment (start 154.305 90.805) (end 160.655 90.805) (width 0.6) (layer F.Cu) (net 3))
 (segment (start 160.655 90.805) (end 162.56 90.805) (width 0.6) (layer F.Cu) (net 3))
 (segment (start 160.655 89.535) (end 160.655 90.805) (width 0.6) (layer F.Cu) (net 3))
 (segment (start 153.14859 89.64859) (end 154.305 90.805) (width 0.6) (layer F.Cu) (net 3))
 (segment (start 153.035 89.64859) (end 153.14859 89.64859) (width 0.6) (layer F.Cu) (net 3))
 (segment (start 166.37 104.775) (end 167.005 104.14) (width 0.6) (layer F.Cu) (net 3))
 (segment (start 167.005 104.14) (end 167.005 93.98) (width 0.6) (layer F.Cu) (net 3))
 (segment (start 167.005 93.98) (end 170.815 90.17) (width 0.6) (layer F.Cu) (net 3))
 (segment (start 170.815 90.17) (end 170.815 86.995) (width 0.6) (layer F.Cu) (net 3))
 (segment (start 170.815 86.995) (end 173.355 84.455) (width 0.6) (layer F.Cu) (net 3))
 (segment (start 173.355 86.995) (end 172.355001 87.994999) (width 0.6) (layer B.Cu) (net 3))
 (segment (start 172.355001 87.994999) (end 172.355001 88.629999) (width 0.6) (layer B.Cu) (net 3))
 (segment (start 172.355001 88.629999) (end 167.005 93.98) (width 0.6) (layer B.Cu) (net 3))
 (segment (start 167.005 93.98) (end 160.655 93.98) (width 0.6) (layer B.Cu) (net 3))
 (segment (start 160.655 93.98) (end 160.655 89.535) (width 0.6) (layer B.Cu) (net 3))
 (via (at 173.355 86.995) (size 2) (drill 1.2) (layers F.Cu B.Cu) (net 3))
 (segment (start 173.355 84.455) (end 173.355 86.995) (width 0.6) (layer F.Cu) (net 3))
 (via (at 160.655 89.535) (size 2) (drill 1.2) (layers F.Cu B.Cu) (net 3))
 (segment (start 153.035 89.64859) (end 153.035 86.995) (width 0.6) (layer F.Cu) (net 3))
 (segment (start 137.16 101.02) (end 137.16 88.265) (width 0.6) (layer F.Cu) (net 3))
 (segment (start 135.255 84.455) (end 135.255 85.997808) (width 0.6) (layer F.Cu) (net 3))
 (segment (start 135.255 85.997808) (end 137.16 87.902808) (width 0.6) (layer F.Cu) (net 3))
 (segment (start 137.16 87.902808) (end 137.16 88.265) (width 0.6) (layer F.Cu) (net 3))
 (segment (start 153.035 84.455) (end 143.51 84.455) (width 0.6) (layer F.Cu) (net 3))
 (segment (start 143.51 84.455) (end 141.605 82.55) (width 0.6) (layer F.Cu) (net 3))
 (segment (start 141.605 82.55) (end 135.89 82.55) (width 0.6) (layer F.Cu) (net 3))
 (segment (start 135.89 82.55) (end 135.255 83.185) (width 0.6) (layer F.Cu) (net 3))
 (segment (start 135.255 83.185) (end 135.255 84.455) (width 0.6) (layer F.Cu) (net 3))
 (segment (start 153.035 86.995) (end 153.035 84.455) (width 0.6) (layer F.Cu) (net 3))
 (segment (start 123.825 112.588908) (end 134.426092 112.588908) (width 0.6) (layer F.Cu) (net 3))
 (segment (start 134.426092 112.588908) (end 134.62 112.395) (width 0.6) (layer F.Cu) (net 3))
 (segment (start 134.62 116.205) (end 134.62 112.395) (width 0.6) (layer F.Cu) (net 3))
 (segment (start 134.62 112.395) (end 134.62 108.67) (width 0.6) (layer F.Cu) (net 3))
 (segment (start 123.172192 110.5361) (end 123.172192 111.9361) (width 0.6) (layer F.Cu) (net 3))
 (segment (start 123.172192 111.9361) (end 123.825 112.588908) (width 0.6) (layer F.Cu) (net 3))
 (segment (start 135.16 102.87) (end 135.31 102.87) (width 0.6) (layer F.Cu) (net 3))
 (segment (start 135.31 102.87) (end 137.16 101.02) (width 0.6) (layer F.Cu) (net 3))
 (segment (start 134.765 102.475) (end 135.16 102.87) (width 0.6) (layer F.Cu) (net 3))
 (segment (start 135.16 106.68) (end 135.16 108.13) (width 0.6) (layer F.Cu) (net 3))
 (segment (start 135.16 108.13) (end 134.62 108.67) (width 0.6) (layer F.Cu) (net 3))
 (segment (start 134.62 116.205) (end 135.285 116.87) (width 0.6) (layer F.Cu) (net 3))
 (segment (start 135.16 102.87) (end 135.16 106.68) (width 0.6) (layer F.Cu) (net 3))
 (segment (start 123.172192 110.5361) (end 123.172192 107.6361) (width 0.6) (layer F.Cu) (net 3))
 (segment (start 123.172192 107.6361) (end 122.657192 107.1211) (width 0.6) (layer F.Cu) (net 3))
 (segment (start 143.51 116.87) (end 135.285 116.87) (width 0.6) (layer F.Cu) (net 3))
 (segment (start 141.478 87.122) (end 141.41958 87.122) (width 0.6) (layer F.Cu) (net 5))
 (segment (start 141.41958 87.122) (end 138.75258 84.455) (width 0.6) (layer F.Cu) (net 5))
 (segment (start 141.478 87.122) (end 141.478 100.584) (width 0.6) (layer F.Cu) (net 5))
 (segment (start 145.035 110.87) (end 143.51 110.87) (width 0.6) (layer F.Cu) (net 5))
 (segment (start 141.478 100.584) (end 141.986 101.092) (width 0.6) (layer F.Cu) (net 5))
 (segment (start 145.415 110.49) (end 145.035 110.87) (width 0.6) (layer F.Cu) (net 5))
 (segment (start 141.986 101.092) (end 145.415 101.092) (width 0.6) (layer F.Cu) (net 5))
 (segment (start 145.415 101.092) (end 145.415 110.49) (width 0.6) (layer F.Cu) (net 5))
 (segment (start 143.51 110.87) (end 142.58 110.87) (width 0.6) (layer F.Cu) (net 5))
 (segment (start 142.58 110.87) (end 142.325 111.125) (width 0.6) (layer F.Cu) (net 5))
 (segment (start 137.795 113.03) (end 137.795 114.205) (width 0.6) (layer F.Cu) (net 5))
 (segment (start 142.325 111.125) (end 139.7 111.125) (width 0.6) (layer F.Cu) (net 5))
 (segment (start 137.795 114.205) (end 137.16 114.84) (width 0.6) (layer F.Cu) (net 5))
 (segment (start 139.7 111.125) (end 137.795 113.03) (width 0.6) (layer F.Cu) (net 5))
 (segment (start 165.989 85.09) (end 167.513 86.614) (width 0.6) (layer F.Cu) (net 6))
 (segment (start 167.513 86.614) (end 167.513 89.535) (width 0.6) (layer F.Cu) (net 6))
 (segment (start 167.513 89.535) (end 163.83 93.218) (width 0.6) (layer F.Cu) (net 6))
 (segment (start 163.83 93.218) (end 163.83 102.235) (width 0.6) (layer F.Cu) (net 6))
 (segment (start 163.83 102.235) (end 159.195 106.87) (width 0.6) (layer F.Cu) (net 6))
 (segment (start 159.195 106.87) (end 157.51 106.87) (width 0.6) (layer F.Cu) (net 6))
 (segment (start 170.815 84.455) (end 168.91 82.55) (width 0.6) (layer F.Cu) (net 6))
 (segment (start 168.91 82.55) (end 167.005 82.55) (width 0.6) (layer F.Cu) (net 6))
 (segment (start 167.005 82.55) (end 165.989 83.566) (width 0.6) (layer F.Cu) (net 6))
 (segment (start 165.989 83.566) (end 165.989 85.09) (width 0.6) (layer F.Cu) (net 6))
 (segment (start 165.989 85.09) (end 163.83 85.09) (width 0.6) (layer F.Cu) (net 6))
 (segment (start 164.465 104.14) (end 164.465 103.378) (width 0.6) (layer F.Cu) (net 7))
 (segment (start 157.51 108.87) (end 159.735 108.87) (width 0.6) (layer F.Cu) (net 7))
 (segment (start 159.735 108.87) (end 164.465 104.14) (width 0.6) (layer F.Cu) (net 7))
 (segment (start 165.481 93.599) (end 168.91 90.17) (width 0.6) (layer F.Cu) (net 7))
 (segment (start 168.91 90.17) (end 168.91 89.535) (width 0.6) (layer F.Cu) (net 7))
 (segment (start 165.481 102.362) (end 165.481 93.599) (width 0.6) (layer F.Cu) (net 7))
 (segment (start 164.465 103.378) (end 165.481 102.362) (width 0.6) (layer F.Cu) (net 7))
 (segment (start 168.91 85.09) (end 168.275 84.455) (width 0.6) (layer F.Cu) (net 7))
 (segment (start 168.91 86.419077) (end 168.91 85.09) (width 0.6) (layer F.Cu) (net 7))
 (segment (start 168.91 86.419077) (end 168.91 87.63) (width 0.6) (layer F.Cu) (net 7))
 (segment (start 163.83 87.63) (end 165.873616 87.63) (width 0.6) (layer F.Cu) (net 7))
 (segment (start 165.873616 87.63) (end 165.941808 87.698192) (width 0.6) (layer F.Cu) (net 7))
 (segment (start 168.91 86.419077) (end 168.91 89.535) (width 0.6) (layer F.Cu) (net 7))
 (segment (start 157.51 104.87) (end 159.29 104.87) (width 0.6) (layer F.Cu) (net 9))
 (segment (start 160.655 92.075) (end 151.13 92.075) (width 0.6) (layer F.Cu) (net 9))
 (segment (start 159.29 104.87) (end 162.56 101.6) (width 0.6) (layer F.Cu) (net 9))
 (segment (start 162.56 101.6) (end 162.56 93.98) (width 0.6) (layer F.Cu) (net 9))
 (segment (start 162.56 93.98) (end 160.655 92.075) (width 0.6) (layer F.Cu) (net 9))
 (segment (start 151.13 92.075) (end 150.495 91.44) (width 0.6) (layer F.Cu) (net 9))
 (segment (start 150.495 91.44) (end 150.495 86.995) (width 0.6) (layer F.Cu) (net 9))
 (segment (start 147.955 86.995) (end 147.955 92.075) (width 0.6) (layer F.Cu) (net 10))
 (segment (start 157.51 102.87) (end 158.75 102.87) (width 0.6) (layer F.Cu) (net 10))
 (segment (start 158.75 102.87) (end 160.655 100.965) (width 0.6) (layer F.Cu) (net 10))
 (segment (start 160.655 100.965) (end 160.655 93.98) (width 0.6) (layer F.Cu) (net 10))
 (segment (start 160.655 93.98) (end 160.02 93.345) (width 0.6) (layer F.Cu) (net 10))
 (segment (start 160.02 93.345) (end 149.225 93.345) (width 0.6) (layer F.Cu) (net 10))
 (segment (start 149.225 93.345) (end 147.955 92.075) (width 0.6) (layer F.Cu) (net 10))
 (segment (start 139.16 102.87) (end 139.16 99.473) (width 0.6) (layer F.Cu) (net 12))
 (segment (start 139.16 99.473) (end 139.446 99.187) (width 0.6) (layer F.Cu) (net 12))
 (segment (start 139.16 102.87) (end 143.51 102.87) (width 0.6) (layer F.Cu) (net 12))
 (segment (start 139.16 106.68) (end 143.32 106.68) (width 0.6) (layer F.Cu) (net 13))
 (segment (start 143.32 106.68) (end 143.51 106.87) (width 0.6) (layer F.Cu) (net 13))
 (segment (start 157.51 114.87) (end 159.895 114.87) (width 0.6) (layer F.Cu) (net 14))
 (segment (start 159.895 114.87) (end 161.925 112.84) (width 0.6) (layer F.Cu) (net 14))
 (segment (start 167.005 110.87) (end 167.005 109.41) (width 0.6) (layer F.Cu) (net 15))
 (segment (start 167.005 109.41) (end 166.37 108.775) (width 0.6) (layer F.Cu) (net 15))
 (segment (start 165.48 110.87) (end 167.005 110.87) (width 0.6) (layer F.Cu) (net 15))
 (segment (start 167.005 112.395) (end 167.005 110.87) (width 0.6) (layer F.Cu) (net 15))
 (segment (start 164.465 118.18056) (end 167.005 115.64056) (width 0.6) (layer F.Cu) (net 15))
 (segment (start 157.51 110.87) (end 165.48 110.87) (width 0.6) (layer F.Cu) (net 15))
 (segment (start 167.005 112.395) (end 167.005 115.64056) (width 0.6) (layer F.Cu) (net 15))
 (segment (start 164.465 119.38) (end 164.465 118.18056) (width 0.6) (layer F.Cu) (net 15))
 (segment (start 157.765 111.125) (end 157.51 110.87) (width 0.6) (layer F.Cu) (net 15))
 (segment (start 157.89 110.49) (end 157.51 110.87) (width 0.6) (layer F.Cu) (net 15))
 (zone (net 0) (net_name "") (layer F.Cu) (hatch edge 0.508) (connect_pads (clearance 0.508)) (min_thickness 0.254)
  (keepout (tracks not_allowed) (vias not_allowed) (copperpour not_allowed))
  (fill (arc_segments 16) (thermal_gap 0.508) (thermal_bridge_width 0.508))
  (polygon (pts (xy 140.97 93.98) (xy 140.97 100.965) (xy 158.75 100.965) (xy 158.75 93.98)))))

